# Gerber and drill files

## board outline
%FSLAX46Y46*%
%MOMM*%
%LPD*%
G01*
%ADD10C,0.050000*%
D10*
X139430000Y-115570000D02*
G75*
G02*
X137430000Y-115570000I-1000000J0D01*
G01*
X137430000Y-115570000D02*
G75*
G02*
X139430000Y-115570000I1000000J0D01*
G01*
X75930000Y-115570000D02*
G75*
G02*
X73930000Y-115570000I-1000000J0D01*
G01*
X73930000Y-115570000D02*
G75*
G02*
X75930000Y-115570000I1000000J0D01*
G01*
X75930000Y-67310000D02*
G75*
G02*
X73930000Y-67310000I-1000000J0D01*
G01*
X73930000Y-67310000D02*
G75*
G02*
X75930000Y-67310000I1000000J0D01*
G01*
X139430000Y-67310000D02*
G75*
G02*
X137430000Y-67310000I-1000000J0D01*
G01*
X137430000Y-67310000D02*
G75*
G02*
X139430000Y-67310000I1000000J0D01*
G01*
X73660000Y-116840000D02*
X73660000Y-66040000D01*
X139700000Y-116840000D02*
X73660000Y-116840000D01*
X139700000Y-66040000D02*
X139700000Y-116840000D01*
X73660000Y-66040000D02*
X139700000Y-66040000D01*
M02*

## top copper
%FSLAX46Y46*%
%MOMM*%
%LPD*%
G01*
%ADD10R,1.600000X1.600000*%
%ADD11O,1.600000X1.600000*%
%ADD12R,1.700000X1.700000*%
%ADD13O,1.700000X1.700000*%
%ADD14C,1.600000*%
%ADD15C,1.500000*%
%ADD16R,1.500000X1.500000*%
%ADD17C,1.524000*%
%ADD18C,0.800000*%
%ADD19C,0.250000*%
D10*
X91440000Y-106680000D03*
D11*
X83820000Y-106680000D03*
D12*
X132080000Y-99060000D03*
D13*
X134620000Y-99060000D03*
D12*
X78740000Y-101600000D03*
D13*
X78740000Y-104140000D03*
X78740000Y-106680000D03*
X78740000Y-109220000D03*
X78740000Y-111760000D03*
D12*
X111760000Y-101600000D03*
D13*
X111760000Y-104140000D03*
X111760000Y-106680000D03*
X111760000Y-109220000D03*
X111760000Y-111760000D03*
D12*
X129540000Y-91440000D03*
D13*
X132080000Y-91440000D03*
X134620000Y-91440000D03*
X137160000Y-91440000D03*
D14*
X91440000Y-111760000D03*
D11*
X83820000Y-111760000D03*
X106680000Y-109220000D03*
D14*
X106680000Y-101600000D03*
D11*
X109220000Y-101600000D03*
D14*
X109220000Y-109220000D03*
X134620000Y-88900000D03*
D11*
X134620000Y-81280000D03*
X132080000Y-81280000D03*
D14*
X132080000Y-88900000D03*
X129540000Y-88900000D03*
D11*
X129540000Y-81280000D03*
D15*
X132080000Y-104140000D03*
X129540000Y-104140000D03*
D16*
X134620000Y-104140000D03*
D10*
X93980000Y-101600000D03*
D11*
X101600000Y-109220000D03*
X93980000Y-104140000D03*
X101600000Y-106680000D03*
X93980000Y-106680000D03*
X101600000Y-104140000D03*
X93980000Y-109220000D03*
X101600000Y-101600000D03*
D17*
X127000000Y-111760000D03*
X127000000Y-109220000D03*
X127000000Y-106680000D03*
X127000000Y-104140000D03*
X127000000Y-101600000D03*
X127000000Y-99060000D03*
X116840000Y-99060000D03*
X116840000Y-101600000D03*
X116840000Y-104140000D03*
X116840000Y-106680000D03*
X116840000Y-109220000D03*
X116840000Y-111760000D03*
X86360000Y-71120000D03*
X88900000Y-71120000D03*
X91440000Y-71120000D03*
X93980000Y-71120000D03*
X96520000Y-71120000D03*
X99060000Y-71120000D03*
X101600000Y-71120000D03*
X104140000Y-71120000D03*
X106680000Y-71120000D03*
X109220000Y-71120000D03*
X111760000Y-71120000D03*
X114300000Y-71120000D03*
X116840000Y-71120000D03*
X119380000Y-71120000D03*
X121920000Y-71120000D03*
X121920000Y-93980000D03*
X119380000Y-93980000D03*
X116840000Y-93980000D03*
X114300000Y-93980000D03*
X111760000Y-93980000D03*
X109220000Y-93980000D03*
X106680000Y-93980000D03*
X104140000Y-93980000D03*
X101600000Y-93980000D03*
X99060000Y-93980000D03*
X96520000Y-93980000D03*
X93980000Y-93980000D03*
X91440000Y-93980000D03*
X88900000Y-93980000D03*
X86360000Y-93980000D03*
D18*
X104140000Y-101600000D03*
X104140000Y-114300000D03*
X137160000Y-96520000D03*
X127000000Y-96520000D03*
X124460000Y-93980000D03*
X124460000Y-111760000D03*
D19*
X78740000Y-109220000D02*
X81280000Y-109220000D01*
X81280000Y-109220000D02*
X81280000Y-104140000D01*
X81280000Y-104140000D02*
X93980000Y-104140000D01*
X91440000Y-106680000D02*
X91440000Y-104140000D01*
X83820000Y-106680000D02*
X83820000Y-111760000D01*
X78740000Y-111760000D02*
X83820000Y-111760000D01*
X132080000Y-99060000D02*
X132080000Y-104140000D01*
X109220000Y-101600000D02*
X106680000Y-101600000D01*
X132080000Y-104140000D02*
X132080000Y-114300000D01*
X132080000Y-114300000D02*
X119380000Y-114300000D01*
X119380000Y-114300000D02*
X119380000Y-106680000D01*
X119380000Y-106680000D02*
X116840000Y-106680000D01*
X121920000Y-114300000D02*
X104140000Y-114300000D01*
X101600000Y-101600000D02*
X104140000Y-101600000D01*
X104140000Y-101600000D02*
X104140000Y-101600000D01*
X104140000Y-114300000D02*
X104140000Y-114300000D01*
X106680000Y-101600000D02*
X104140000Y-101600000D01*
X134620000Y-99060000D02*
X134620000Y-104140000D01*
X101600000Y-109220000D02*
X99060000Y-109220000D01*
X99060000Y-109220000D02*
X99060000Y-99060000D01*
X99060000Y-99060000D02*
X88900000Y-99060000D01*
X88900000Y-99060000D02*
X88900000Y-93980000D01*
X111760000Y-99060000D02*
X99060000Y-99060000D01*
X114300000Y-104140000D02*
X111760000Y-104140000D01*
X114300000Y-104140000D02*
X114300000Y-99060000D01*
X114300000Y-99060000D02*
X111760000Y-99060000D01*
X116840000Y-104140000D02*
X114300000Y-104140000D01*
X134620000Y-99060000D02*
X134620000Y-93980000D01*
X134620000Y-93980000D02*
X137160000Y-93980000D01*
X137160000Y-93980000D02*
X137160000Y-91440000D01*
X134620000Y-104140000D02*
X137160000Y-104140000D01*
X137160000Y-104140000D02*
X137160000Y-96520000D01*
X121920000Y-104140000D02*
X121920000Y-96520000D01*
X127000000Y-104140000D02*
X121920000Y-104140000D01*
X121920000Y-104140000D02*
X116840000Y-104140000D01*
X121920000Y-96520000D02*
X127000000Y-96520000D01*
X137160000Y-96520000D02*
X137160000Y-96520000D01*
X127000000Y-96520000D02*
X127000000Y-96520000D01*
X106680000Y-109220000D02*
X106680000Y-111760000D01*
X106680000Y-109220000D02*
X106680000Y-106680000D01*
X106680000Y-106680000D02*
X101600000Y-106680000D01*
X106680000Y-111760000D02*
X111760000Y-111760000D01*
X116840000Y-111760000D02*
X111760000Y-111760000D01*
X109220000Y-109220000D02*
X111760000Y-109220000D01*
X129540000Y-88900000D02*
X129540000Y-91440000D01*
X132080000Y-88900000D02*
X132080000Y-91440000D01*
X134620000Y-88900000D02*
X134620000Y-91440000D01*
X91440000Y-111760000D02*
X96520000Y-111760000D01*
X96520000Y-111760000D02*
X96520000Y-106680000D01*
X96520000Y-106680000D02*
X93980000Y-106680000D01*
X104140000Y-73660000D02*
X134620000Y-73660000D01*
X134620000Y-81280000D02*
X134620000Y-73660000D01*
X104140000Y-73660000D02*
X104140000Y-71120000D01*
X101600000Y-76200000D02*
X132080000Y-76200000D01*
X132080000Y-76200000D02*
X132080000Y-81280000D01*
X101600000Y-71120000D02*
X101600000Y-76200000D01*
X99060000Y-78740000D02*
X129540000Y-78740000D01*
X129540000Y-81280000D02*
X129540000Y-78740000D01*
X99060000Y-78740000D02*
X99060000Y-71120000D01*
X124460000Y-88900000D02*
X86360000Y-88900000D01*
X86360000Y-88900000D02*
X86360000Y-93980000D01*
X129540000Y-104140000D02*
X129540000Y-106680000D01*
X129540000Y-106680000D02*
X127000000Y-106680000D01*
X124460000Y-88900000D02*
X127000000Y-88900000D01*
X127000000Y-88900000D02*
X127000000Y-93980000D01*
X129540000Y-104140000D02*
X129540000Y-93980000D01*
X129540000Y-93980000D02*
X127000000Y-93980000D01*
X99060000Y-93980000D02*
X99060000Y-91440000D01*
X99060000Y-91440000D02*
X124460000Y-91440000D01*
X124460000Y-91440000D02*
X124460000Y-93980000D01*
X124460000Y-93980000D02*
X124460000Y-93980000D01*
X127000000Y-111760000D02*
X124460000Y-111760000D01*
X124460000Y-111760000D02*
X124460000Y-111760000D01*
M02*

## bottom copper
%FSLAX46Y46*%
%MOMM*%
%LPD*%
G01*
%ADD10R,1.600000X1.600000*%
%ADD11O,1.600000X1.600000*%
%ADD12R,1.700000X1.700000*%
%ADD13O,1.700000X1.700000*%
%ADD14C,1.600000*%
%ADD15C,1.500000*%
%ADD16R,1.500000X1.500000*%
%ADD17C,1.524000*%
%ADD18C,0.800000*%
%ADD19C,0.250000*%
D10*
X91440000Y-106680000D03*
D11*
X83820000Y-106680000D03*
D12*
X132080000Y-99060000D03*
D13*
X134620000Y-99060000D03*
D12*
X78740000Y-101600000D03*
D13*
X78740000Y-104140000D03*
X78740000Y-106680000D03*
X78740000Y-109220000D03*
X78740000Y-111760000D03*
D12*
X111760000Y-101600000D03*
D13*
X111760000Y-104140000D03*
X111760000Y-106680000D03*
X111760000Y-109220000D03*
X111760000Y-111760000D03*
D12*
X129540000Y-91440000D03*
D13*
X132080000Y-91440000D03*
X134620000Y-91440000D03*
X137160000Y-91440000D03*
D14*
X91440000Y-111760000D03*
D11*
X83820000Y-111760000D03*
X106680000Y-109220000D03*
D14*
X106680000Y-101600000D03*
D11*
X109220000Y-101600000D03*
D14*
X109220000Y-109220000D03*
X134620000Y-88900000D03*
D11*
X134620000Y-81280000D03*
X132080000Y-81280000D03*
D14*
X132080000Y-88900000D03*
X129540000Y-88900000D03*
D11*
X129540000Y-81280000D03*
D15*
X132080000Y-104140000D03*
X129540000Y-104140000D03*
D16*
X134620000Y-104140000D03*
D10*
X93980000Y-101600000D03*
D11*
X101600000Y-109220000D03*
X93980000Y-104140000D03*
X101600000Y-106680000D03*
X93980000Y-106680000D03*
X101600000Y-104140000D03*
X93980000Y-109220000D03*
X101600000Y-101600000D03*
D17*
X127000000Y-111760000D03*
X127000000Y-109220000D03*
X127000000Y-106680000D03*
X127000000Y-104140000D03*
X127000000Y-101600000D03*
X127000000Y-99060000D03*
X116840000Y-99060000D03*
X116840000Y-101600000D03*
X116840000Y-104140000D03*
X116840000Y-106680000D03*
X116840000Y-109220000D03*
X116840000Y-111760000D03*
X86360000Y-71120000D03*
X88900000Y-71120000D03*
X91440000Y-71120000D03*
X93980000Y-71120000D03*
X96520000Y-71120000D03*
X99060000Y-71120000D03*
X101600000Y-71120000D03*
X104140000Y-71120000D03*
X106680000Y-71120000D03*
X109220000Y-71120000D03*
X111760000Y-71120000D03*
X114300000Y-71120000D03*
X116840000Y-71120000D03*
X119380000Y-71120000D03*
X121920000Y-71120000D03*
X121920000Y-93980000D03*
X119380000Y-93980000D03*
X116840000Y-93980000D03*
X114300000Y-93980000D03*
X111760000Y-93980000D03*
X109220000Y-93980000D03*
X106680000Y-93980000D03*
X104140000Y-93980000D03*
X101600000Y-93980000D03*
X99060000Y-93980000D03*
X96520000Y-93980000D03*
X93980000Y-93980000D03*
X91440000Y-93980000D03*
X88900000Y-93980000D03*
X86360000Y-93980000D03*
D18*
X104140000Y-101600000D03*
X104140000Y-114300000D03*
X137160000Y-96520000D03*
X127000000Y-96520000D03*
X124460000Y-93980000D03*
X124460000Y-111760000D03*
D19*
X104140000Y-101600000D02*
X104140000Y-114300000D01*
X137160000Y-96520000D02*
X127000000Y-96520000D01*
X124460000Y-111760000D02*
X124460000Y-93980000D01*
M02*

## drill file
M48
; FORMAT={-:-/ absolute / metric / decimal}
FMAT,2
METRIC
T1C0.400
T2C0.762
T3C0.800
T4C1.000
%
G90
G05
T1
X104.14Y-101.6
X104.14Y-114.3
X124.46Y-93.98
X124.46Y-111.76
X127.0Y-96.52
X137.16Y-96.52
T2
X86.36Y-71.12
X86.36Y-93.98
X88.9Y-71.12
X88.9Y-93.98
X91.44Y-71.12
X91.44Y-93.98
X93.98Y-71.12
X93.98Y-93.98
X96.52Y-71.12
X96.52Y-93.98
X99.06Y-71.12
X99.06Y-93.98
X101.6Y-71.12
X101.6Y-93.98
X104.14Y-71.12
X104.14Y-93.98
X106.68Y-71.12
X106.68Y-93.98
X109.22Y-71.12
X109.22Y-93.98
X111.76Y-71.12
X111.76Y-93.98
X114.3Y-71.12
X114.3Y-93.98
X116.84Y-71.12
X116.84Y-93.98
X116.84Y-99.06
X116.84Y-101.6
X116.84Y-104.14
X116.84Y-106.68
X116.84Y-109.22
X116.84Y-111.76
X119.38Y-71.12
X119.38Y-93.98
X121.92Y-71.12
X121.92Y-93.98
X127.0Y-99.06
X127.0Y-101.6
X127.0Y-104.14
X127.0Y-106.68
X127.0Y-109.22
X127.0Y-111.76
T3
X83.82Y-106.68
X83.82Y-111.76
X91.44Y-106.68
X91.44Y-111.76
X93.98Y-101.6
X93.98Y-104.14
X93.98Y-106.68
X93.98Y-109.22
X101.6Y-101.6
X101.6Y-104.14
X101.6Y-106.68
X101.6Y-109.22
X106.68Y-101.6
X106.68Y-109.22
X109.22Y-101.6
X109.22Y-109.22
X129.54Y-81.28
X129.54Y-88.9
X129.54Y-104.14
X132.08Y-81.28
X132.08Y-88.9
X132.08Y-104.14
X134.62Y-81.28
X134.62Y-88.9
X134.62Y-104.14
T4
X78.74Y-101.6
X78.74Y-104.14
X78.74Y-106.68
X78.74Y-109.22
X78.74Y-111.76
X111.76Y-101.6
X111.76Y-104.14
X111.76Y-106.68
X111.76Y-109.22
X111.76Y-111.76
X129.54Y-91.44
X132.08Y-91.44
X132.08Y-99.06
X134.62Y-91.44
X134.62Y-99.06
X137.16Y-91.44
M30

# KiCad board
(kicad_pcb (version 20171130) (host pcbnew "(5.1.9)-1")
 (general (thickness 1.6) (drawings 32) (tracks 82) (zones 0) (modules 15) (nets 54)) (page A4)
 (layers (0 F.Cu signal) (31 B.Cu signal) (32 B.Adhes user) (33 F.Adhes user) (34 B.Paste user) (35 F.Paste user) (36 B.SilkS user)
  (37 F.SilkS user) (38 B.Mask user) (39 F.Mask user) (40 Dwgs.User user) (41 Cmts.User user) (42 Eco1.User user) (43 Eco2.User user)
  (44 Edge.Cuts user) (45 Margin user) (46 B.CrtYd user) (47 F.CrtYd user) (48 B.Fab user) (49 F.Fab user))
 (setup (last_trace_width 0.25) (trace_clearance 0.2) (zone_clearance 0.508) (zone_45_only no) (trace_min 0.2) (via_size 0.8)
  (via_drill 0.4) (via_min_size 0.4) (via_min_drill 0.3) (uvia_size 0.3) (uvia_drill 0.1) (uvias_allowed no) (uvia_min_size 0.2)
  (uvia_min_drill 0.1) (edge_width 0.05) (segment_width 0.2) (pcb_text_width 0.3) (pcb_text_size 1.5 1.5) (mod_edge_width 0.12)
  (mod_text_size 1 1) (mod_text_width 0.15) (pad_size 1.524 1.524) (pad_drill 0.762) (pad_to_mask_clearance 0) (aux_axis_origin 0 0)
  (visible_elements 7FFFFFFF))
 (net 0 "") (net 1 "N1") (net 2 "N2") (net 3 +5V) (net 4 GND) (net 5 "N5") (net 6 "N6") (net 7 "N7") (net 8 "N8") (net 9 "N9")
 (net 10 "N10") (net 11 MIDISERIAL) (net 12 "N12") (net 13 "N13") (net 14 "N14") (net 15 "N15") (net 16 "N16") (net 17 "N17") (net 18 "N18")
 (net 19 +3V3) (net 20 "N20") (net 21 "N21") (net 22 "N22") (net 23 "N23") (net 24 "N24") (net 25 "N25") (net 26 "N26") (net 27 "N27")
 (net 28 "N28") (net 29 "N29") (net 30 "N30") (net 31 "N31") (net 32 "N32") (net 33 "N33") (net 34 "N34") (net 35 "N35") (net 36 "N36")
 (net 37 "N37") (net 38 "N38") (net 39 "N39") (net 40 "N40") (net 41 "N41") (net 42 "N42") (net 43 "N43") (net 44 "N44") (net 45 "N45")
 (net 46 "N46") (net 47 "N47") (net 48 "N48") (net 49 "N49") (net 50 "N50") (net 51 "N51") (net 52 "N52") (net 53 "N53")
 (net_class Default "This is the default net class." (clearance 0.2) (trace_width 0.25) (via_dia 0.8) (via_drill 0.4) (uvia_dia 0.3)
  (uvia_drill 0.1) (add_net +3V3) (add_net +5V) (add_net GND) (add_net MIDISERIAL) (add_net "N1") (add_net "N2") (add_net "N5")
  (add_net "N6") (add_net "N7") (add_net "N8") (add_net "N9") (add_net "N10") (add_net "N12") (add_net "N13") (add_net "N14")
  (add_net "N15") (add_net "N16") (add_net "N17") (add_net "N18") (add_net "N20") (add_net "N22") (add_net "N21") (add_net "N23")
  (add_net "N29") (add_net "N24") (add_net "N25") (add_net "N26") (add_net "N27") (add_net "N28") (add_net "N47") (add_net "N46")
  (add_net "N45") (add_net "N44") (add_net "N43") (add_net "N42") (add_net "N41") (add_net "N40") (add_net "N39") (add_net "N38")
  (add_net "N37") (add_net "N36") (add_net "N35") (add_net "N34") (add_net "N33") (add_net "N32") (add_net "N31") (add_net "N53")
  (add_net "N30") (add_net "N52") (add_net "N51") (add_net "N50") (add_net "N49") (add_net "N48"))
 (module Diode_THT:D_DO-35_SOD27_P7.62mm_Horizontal (layer F.Cu) (at 91.44 106.68 180)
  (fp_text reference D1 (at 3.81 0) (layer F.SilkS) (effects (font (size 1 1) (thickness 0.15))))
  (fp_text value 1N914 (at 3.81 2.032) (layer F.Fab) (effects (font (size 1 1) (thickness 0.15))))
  (pad 1 thru_hole rect (at 0 0 180) (size 1.6 1.6) (drill 0.8) (layers *.Cu *.Mask) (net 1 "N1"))
  (pad 2 thru_hole oval (at 7.62 0 180) (size 1.6 1.6) (drill 0.8) (layers *.Cu *.Mask) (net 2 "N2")))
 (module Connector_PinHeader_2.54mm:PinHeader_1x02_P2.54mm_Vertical (layer F.Cu) (at 132.08 99.06 90)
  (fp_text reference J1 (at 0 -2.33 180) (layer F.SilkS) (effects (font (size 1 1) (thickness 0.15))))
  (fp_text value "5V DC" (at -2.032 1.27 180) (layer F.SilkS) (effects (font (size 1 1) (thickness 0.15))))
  (pad 1 thru_hole rect (at 0 0 90) (size 1.7 1.7) (drill 1) (layers *.Cu *.Mask) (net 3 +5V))
  (pad 2 thru_hole oval (at 0 2.54 90) (size 1.7 1.7) (drill 1) (layers *.Cu *.Mask) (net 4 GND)))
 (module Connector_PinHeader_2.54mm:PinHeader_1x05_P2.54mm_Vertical (layer F.Cu) (at 78.74 101.6)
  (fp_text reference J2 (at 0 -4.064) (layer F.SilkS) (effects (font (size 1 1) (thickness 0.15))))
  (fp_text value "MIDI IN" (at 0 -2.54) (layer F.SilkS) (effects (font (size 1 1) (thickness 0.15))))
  (pad 1 thru_hole rect (at 0 0) (size 1.7 1.7) (drill 1) (layers *.Cu *.Mask) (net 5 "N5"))
  (pad 2 thru_hole oval (at 0 2.54) (size 1.7 1.7) (drill 1) (layers *.Cu *.Mask) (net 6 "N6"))
  (pad 3 thru_hole oval (at 0 5.08) (size 1.7 1.7) (drill 1) (layers *.Cu *.Mask) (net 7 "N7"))
  (pad 4 thru_hole oval (at 0 7.62) (size 1.7 1.7) (drill 1) (layers *.Cu *.Mask) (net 1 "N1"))
  (pad 5 thru_hole oval (at 0 10.16) (size 1.7 1.7) (drill 1) (layers *.Cu *.Mask) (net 2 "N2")))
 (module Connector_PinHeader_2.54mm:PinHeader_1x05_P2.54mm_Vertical (layer F.Cu) (at 111.76 101.6)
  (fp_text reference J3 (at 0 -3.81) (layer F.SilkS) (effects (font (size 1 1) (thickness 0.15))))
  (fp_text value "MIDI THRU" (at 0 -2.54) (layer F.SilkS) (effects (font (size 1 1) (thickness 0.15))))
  (pad 1 thru_hole rect (at 0 0) (size 1.7 1.7) (drill 1) (layers *.Cu *.Mask) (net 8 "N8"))
  (pad 2 thru_hole oval (at 0 2.54) (size 1.7 1.7) (drill 1) (layers *.Cu *.Mask) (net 4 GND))
  (pad 3 thru_hole oval (at 0 5.08) (size 1.7 1.7) (drill 1) (layers *.Cu *.Mask) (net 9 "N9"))
  (pad 4 thru_hole oval (at 0 7.62) (size 1.7 1.7) (drill 1) (layers *.Cu *.Mask) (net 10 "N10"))
  (pad 5 thru_hole oval (at 0 10.16) (size 1.7 1.7) (drill 1) (layers *.Cu *.Mask) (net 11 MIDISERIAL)))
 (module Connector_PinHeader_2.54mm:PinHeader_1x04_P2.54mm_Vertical (layer F.Cu) (at 129.54 91.44 90)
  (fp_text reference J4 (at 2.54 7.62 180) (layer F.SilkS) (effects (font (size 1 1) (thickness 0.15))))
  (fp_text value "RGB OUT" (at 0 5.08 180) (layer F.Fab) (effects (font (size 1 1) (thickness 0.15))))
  (pad 1 thru_hole rect (at 0 0 90) (size 1.7 1.7) (drill 1) (layers *.Cu *.Mask) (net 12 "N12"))
  (pad 2 thru_hole oval (at 0 2.54 90) (size 1.7 1.7) (drill 1) (layers *.Cu *.Mask) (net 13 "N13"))
  (pad 3 thru_hole oval (at 0 5.08 90) (size 1.7 1.7) (drill 1) (layers *.Cu *.Mask) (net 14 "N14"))
  (pad 4 thru_hole oval (at 0 7.62 90) (size 1.7 1.7) (drill 1) (layers *.Cu *.Mask) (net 4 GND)))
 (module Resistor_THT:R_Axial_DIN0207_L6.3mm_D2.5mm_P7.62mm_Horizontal (layer F.Cu) (at 91.44 111.76 180)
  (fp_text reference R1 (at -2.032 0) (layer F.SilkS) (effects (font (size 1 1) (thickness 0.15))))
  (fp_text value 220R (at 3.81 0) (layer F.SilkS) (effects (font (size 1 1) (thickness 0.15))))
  (pad 1 thru_hole circle (at 0 0 180) (size 1.6 1.6) (drill 0.8) (layers *.Cu *.Mask) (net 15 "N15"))
  (pad 2 thru_hole oval (at 7.62 0 180) (size 1.6 1.6) (drill 0.8) (layers *.Cu *.Mask) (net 2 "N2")))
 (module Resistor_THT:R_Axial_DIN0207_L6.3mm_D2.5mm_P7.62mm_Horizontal (layer F.Cu) (at 106.68 101.6 270)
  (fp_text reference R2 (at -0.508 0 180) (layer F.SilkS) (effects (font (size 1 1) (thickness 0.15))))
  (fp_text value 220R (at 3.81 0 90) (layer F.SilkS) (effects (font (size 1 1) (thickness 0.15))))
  (pad 2 thru_hole oval (at 7.62 0 270) (size 1.6 1.6) (drill 0.8) (layers *.Cu *.Mask) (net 11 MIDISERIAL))
  (pad 1 thru_hole circle (at 0 0 270) (size 1.6 1.6) (drill 0.8) (layers *.Cu *.Mask) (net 3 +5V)))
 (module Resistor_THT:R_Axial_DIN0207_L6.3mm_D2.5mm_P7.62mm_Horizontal (layer F.Cu) (at 109.22 109.22 90)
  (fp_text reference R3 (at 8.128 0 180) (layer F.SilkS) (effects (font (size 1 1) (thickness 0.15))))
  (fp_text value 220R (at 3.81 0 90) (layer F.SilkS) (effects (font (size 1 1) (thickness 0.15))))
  (pad 2 thru_hole oval (at 7.62 0 90) (size 1.6 1.6) (drill 0.8) (layers *.Cu *.Mask) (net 3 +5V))
  (pad 1 thru_hole circle (at 0 0 90) (size 1.6 1.6) (drill 0.8) (layers *.Cu *.Mask) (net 10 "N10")))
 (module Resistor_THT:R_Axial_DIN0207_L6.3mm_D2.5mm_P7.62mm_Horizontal (layer F.Cu) (at 134.62 88.9 90)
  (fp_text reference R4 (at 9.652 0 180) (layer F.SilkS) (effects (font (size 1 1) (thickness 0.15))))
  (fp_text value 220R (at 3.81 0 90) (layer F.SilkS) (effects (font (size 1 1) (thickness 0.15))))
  (pad 1 thru_hole circle (at 0 0 90) (size 1.6 1.6) (drill 0.8) (layers *.Cu *.Mask) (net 14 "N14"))
  (pad 2 thru_hole oval (at 7.62 0 90) (size 1.6 1.6) (drill 0.8) (layers *.Cu *.Mask) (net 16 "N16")))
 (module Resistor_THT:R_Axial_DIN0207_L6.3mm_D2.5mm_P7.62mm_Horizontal (layer F.Cu) (at 132.08 88.9 90)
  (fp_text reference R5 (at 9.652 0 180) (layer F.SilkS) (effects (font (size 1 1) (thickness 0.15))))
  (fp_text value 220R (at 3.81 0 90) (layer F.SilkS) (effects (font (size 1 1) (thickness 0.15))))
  (pad 2 thru_hole oval (at 7.62 0 90) (size 1.6 1.6) (drill 0.8) (layers *.Cu *.Mask) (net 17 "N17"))
  (pad 1 thru_hole circle (at 0 0 90) (size 1.6 1.6) (drill 0.8) (layers *.Cu *.Mask) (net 13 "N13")))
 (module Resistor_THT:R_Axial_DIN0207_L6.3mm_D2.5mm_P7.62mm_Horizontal (layer F.Cu) (at 129.54 88.9 90)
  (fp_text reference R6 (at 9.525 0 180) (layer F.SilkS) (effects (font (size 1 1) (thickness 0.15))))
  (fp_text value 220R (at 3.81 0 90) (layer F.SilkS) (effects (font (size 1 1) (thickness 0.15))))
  (pad 1 thru_hole circle (at 0 0 90) (size 1.6 1.6) (drill 0.8) (layers *.Cu *.Mask) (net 12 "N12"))
  (pad 2 thru_hole oval (at 7.62 0 90) (size 1.6 1.6) (drill 0.8) (layers *.Cu *.Mask) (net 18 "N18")))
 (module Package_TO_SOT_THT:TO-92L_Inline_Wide (layer F.Cu) (at 134.62 104.14 180)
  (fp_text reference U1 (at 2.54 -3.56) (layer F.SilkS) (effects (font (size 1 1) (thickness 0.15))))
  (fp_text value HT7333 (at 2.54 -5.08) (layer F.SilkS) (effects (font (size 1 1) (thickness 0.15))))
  (pad 2 thru_hole circle (at 2.54 0 180) (size 1.5 1.5) (drill 0.8) (layers *.Cu *.Mask) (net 3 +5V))
  (pad 3 thru_hole circle (at 5.08 0 180) (size 1.5 1.5) (drill 0.8) (layers *.Cu *.Mask) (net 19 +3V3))
  (pad 1 thru_hole rect (at 0 0 180) (size 1.5 1.5) (drill 0.8) (layers *.Cu *.Mask) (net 4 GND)))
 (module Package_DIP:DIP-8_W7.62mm (layer F.Cu) (at 93.98 101.6)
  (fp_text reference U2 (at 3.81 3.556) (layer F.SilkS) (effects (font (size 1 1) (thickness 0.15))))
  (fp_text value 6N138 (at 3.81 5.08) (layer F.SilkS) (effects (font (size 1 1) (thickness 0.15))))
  (pad 1 thru_hole rect (at 0 0) (size 1.6 1.6) (drill 0.8) (layers *.Cu *.Mask) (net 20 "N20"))
  (pad 5 thru_hole oval (at 7.62 7.62) (size 1.6 1.6) (drill 0.8) (layers *.Cu *.Mask) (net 4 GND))
  (pad 2 thru_hole oval (at 0 2.54) (size 1.6 1.6) (drill 0.8) (layers *.Cu *.Mask) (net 1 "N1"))
  (pad 6 thru_hole oval (at 7.62 5.08) (size 1.6 1.6) (drill 0.8) (layers *.Cu *.Mask) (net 11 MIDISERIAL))
  (pad 3 thru_hole oval (at 0 5.08) (size 1.6 1.6) (drill 0.8) (layers *.Cu *.Mask) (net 15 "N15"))
  (pad 7 thru_hole oval (at 7.62 2.54) (size 1.6 1.6) (drill 0.8) (layers *.Cu *.Mask) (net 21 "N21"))
  (pad 4 thru_hole oval (at 0 7.62) (size 1.6 1.6) (drill 0.8) (layers *.Cu *.Mask) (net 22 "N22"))
  (pad 8 thru_hole oval (at 7.62 0) (size 1.6 1.6) (drill 0.8) (layers *.Cu *.Mask) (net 3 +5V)))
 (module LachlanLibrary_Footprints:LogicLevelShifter (layer F.Cu) (at 121.92 105.41 180)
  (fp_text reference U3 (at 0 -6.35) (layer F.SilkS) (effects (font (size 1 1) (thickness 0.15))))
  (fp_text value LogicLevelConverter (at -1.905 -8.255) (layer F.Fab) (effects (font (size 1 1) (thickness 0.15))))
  (pad 1 thru_hole circle (at -5.08 -6.35 180) (size 1.524 1.524) (drill 0.762) (layers *.Cu *.Mask) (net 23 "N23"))
  (pad 2 thru_hole circle (at -5.08 -3.81 180) (size 1.524 1.524) (drill 0.762) (layers *.Cu *.Mask) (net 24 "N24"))
  (pad 3 thru_hole circle (at -5.08 -1.27 180) (size 1.524 1.524) (drill 0.762) (layers *.Cu *.Mask) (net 19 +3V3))
  (pad 4 thru_hole circle (at -5.08 1.27 180) (size 1.524 1.524) (drill 0.762) (layers *.Cu *.Mask) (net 4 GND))
  (pad 5 thru_hole circle (at -5.08 3.81 180) (size 1.524 1.524) (drill 0.762) (layers *.Cu *.Mask) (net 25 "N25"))
  (pad 6 thru_hole circle (at -5.08 6.35 180) (size 1.524 1.524) (drill 0.762) (layers *.Cu *.Mask) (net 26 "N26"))
  (pad 7 thru_hole circle (at 5.08 6.35 180) (size 1.524 1.524) (drill 0.762) (layers *.Cu *.Mask) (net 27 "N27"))
  (pad 8 thru_hole circle (at 5.08 3.81 180) (size 1.524 1.524) (drill 0.762) (layers *.Cu *.Mask) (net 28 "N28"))
  (pad 9 thru_hole circle (at 5.08 1.27 180) (size 1.524 1.524) (drill 0.762) (layers *.Cu *.Mask) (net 4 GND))
  (pad 10 thru_hole circle (at 5.08 -1.27 180) (size 1.524 1.524) (drill 0.762) (layers *.Cu *.Mask) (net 3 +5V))
  (pad 11 thru_hole circle (at 5.08 -3.81 180) (size 1.524 1.524) (drill 0.762) (layers *.Cu *.Mask) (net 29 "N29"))
  (pad 12 thru_hole circle (at 5.08 -6.35 180) (size 1.524 1.524) (drill 0.762) (layers *.Cu *.Mask) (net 11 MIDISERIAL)))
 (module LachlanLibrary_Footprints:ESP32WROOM (layer F.Cu) (at 105.41 82.55 90)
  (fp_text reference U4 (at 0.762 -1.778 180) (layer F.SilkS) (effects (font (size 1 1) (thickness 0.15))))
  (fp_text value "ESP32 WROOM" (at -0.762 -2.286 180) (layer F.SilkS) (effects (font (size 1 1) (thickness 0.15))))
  (pad 30 thru_hole circle (at 11.43 -19.05 90) (size 1.524 1.524) (drill 0.762) (layers *.Cu *.Mask) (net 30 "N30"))
  (pad 29 thru_hole circle (at 11.43 -16.51 90) (size 1.524 1.524) (drill 0.762) (layers *.Cu *.Mask) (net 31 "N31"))
  (pad 28 thru_hole circle (at 11.43 -13.97 90) (size 1.524 1.524) (drill 0.762) (layers *.Cu *.Mask) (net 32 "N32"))
  (pad 27 thru_hole circle (at 11.43 -11.43 90) (size 1.524 1.524) (drill 0.762) (layers *.Cu *.Mask) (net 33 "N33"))
  (pad 26 thru_hole circle (at 11.43 -8.89 90) (size 1.524 1.524) (drill 0.762) (layers *.Cu *.Mask) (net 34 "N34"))
  (pad 25 thru_hole circle (at 11.43 -6.35 90) (size 1.524 1.524) (drill 0.762) (layers *.Cu *.Mask) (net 18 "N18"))
  (pad 24 thru_hole circle (at 11.43 -3.81 90) (size 1.524 1.524) (drill 0.762) (layers *.Cu *.Mask) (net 17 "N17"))
  (pad 23 thru_hole circle (at 11.43 -1.27 90) (size 1.524 1.524) (drill 0.762) (layers *.Cu *.Mask) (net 16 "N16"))
  (pad 22 thru_hole circle (at 11.43 1.27 90) (size 1.524 1.524) (drill 0.762) (layers *.Cu *.Mask) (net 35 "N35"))
  (pad 21 thru_hole circle (at 11.43 3.81 90) (size 1.524 1.524) (drill 0.762) (layers *.Cu *.Mask) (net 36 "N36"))
  (pad 20 thru_hole circle (at 11.43 6.35 90) (size 1.524 1.524) (drill 0.762) (layers *.Cu *.Mask) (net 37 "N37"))
  (pad 19 thru_hole circle (at 11.43 8.89 90) (size 1.524 1.524) (drill 0.762) (layers *.Cu *.Mask) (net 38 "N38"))
  (pad 18 thru_hole circle (at 11.43 11.43 90) (size 1.524 1.524) (drill 0.762) (layers *.Cu *.Mask) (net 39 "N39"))
  (pad 17 thru_hole circle (at 11.43 13.97 90) (size 1.524 1.524) (drill 0.762) (layers *.Cu *.Mask) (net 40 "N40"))
  (pad 16 thru_hole circle (at 11.43 16.51 90) (size 1.524 1.524) (drill 0.762) (layers *.Cu *.Mask) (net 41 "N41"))
  (pad 15 thru_hole circle (at -11.43 16.51 90) (size 1.524 1.524) (drill 0.762) (layers *.Cu *.Mask) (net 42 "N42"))
  (pad 14 thru_hole circle (at -11.43 13.97 90) (size 1.524 1.524) (drill 0.762) (layers *.Cu *.Mask) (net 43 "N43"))
  (pad 13 thru_hole circle (at -11.43 11.43 90) (size 1.524 1.524) (drill 0.762) (layers *.Cu *.Mask) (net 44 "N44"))
  (pad 12 thru_hole circle (at -11.43 8.89 90) (size 1.524 1.524) (drill 0.762) (layers *.Cu *.Mask) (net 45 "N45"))
  (pad 11 thru_hole circle (at -11.43 6.35 90) (size 1.524 1.524) (drill 0.762) (layers *.Cu *.Mask) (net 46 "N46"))
  (pad 10 thru_hole circle (at -11.43 3.81 90) (size 1.524 1.524) (drill 0.762) (layers *.Cu *.Mask) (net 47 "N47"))
  (pad 9 thru_hole circle (at -11.43 1.27 90) (size 1.524 1.524) (drill 0.762) (layers *.Cu *.Mask) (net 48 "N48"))
  (pad 8 thru_hole circle (at -11.43 -1.27 90) (size 1.524 1.524) (drill 0.762) (layers *.Cu *.Mask) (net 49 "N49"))
  (pad 7 thru_hole circle (at -11.43 -3.81 90) (size 1.524 1.524) (drill 0.762) (layers *.Cu *.Mask) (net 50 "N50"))
  (pad 6 thru_hole circle (at -11.43 -6.35 90) (size 1.524 1.524) (drill 0.762) (layers *.Cu *.Mask) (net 23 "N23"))
  (pad 5 thru_hole circle (at -11.43 -8.89 90) (size 1.524 1.524) (drill 0.762) (layers *.Cu *.Mask) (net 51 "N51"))
  (pad 4 thru_hole circle (at -11.43 -11.43 90) (size 1.524 1.524) (drill 0.762) (layers *.Cu *.Mask) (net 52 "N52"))
  (pad 3 thru_hole circle (at -11.43 -13.97 90) (size 1.524 1.524) (drill 0.762) (layers *.Cu *.Mask) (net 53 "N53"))
  (pad 2 thru_hole circle (at -11.43 -16.51 90) (size 1.524 1.524) (drill 0.762) (layers *.Cu *.Mask) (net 4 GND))
  (pad 1 thru_hole circle (at -11.43 -19.05 90) (size 1.524 1.524) (drill 0.762) (layers *.Cu *.Mask) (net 19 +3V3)))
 (gr_circle (center 138.43 115.57) (end 139.43 115.57) (layer Edge.Cuts) (width 0.05))
 (gr_circle (center 74.93 115.57) (end 75.93 115.57) (layer Edge.Cuts) (width 0.05))
 (gr_circle (center 74.93 67.31) (end 75.93 67.31) (layer Edge.Cuts) (width 0.05))
 (gr_circle (center 138.43 67.31) (end 139.43 67.31) (layer Edge.Cuts) (width 0.05))
 (gr_line (start 73.66 116.84) (end 73.66 66.04) (layer Edge.Cuts) (width 0.05))
 (gr_line (start 139.7 116.84) (end 73.66 116.84) (layer Edge.Cuts) (width 0.05))
 (gr_line (start 139.7 66.04) (end 139.7 116.84) (layer Edge.Cuts) (width 0.05))
 (gr_line (start 73.66 66.04) (end 139.7 66.04) (layer Edge.Cuts) (width 0.05))
 (segment (start 78.74 109.22) (end 81.28 109.22) (width 0.25) (layer F.Cu) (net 1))
 (segment (start 81.28 109.22) (end 81.28 104.14) (width 0.25) (layer F.Cu) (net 1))
 (segment (start 81.28 104.14) (end 93.98 104.14) (width 0.25) (layer F.Cu) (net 1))
 (segment (start 91.44 106.68) (end 91.44 104.14) (width 0.25) (layer F.Cu) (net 1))
 (segment (start 83.82 106.68) (end 83.82 111.76) (width 0.25) (layer F.Cu) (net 2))
 (segment (start 78.74 111.76) (end 83.82 111.76) (width 0.25) (layer F.Cu) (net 2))
 (segment (start 132.08 99.06) (end 132.08 104.14) (width 0.25) (layer F.Cu) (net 3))
 (segment (start 109.22 101.6) (end 106.68 101.6) (width 0.25) (layer F.Cu) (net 3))
 (segment (start 132.08 104.14) (end 132.08 114.3) (width 0.25) (layer F.Cu) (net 3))
 (segment (start 132.08 114.3) (end 119.38 114.3) (width 0.25) (layer F.Cu) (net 3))
 (segment (start 119.38 114.3) (end 119.38 106.68) (width 0.25) (layer F.Cu) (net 3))
 (segment (start 119.38 106.68) (end 116.84 106.68) (width 0.25) (layer F.Cu) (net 3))
 (segment (start 121.92 114.3) (end 104.14 114.3) (width 0.25) (layer F.Cu) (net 3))
 (segment (start 101.6 101.6) (end 104.14 101.6) (width 0.25) (layer F.Cu) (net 3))
 (segment (start 104.14 101.6) (end 104.14 101.6) (width 0.25) (layer F.Cu) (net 3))
 (via (at 104.14 101.6) (size 0.8) (drill 0.4) (layers F.Cu B.Cu) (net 3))
 (segment (start 104.14 114.3) (end 104.14 114.3) (width 0.25) (layer F.Cu) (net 3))
 (via (at 104.14 114.3) (size 0.8) (drill 0.4) (layers F.Cu B.Cu) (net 3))
 (segment (start 106.68 101.6) (end 104.14 101.6) (width 0.25) (layer F.Cu) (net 3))
 (segment (start 104.14 101.6) (end 104.14 114.3) (width 0.25) (layer B.Cu) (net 3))
 (segment (start 134.62 99.06) (end 134.62 104.14) (width 0.25) (layer F.Cu) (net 4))
 (segment (start 101.6 109.22) (end 99.06 109.22) (width 0.25) (layer F.Cu) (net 4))
 (segment (start 99.06 109.22) (end 99.06 99.06) (width 0.25) (layer F.Cu) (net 4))
 (segment (start 99.06 99.06) (end 88.9 99.06) (width 0.25) (layer F.Cu) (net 4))
 (segment (start 88.9 99.06) (end 88.9 93.98) (width 0.25) (layer F.Cu) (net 4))
 (segment (start 111.76 99.06) (end 99.06 99.06) (width 0.25) (layer F.Cu) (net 4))
 (segment (start 114.3 104.14) (end 111.76 104.14) (width 0.25) (layer F.Cu) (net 4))
 (segment (start 114.3 104.14) (end 114.3 99.06) (width 0.25) (layer F.Cu) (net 4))
 (segment (start 114.3 99.06) (end 111.76 99.06) (width 0.25) (layer F.Cu) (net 4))
 (segment (start 116.84 104.14) (end 114.3 104.14) (width 0.25) (layer F.Cu) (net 4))
 (segment (start 134.62 99.06) (end 134.62 93.98) (width 0.25) (layer F.Cu) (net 4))
 (segment (start 134.62 93.98) (end 137.16 93.98) (width 0.25) (layer F.Cu) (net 4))
 (segment (start 137.16 93.98) (end 137.16 91.44) (width 0.25) (layer F.Cu) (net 4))
 (segment (start 134.62 104.14) (end 137.16 104.14) (width 0.25) (layer F.Cu) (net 4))
 (segment (start 137.16 104.14) (end 137.16 96.52) (width 0.25) (layer F.Cu) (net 4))
 (segment (start 121.92 104.14) (end 121.92 96.52) (width 0.25) (layer F.Cu) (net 4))
 (segment (start 127 104.14) (end 121.92 104.14) (width 0.25) (layer F.Cu) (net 4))
 (segment (start 121.92 104.14) (end 116.84 104.14) (width 0.25) (layer F.Cu) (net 4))
 (segment (start 121.92 96.52) (end 127 96.52) (width 0.25) (layer F.Cu) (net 4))
 (segment (start 137.16 96.52) (end 137.16 96.52) (width 0.25) (layer F.Cu) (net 4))
 (via (at 137.16 96.52) (size 0.8) (drill 0.4) (layers F.Cu B.Cu) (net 4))
 (segment (start 127 96.52) (end 127 96.52) (width 0.25) (layer F.Cu) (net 4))
 (via (at 127 96.52) (size 0.8) (drill 0.4) (layers F.Cu B.Cu) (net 4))
 (segment (start 137.16 96.52) (end 127 96.52) (width 0.25) (layer B.Cu) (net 4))
 (segment (start 106.68 109.22) (end 106.68 111.76) (width 0.25) (layer F.Cu) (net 11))
 (segment (start 106.68 109.22) (end 106.68 106.68) (width 0.25) (layer F.Cu) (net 11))
 (segment (start 106.68 106.68) (end 101.6 106.68) (width 0.25) (layer F.Cu) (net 11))
 (segment (start 106.68 111.76) (end 111.76 111.76) (width 0.25) (layer F.Cu) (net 11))
 (segment (start 116.84 111.76) (end 111.76 111.76) (width 0.25) (layer F.Cu) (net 11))
 (segment (start 109.22 109.22) (end 111.76 109.22) (width 0.25) (layer F.Cu) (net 10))
 (segment (start 129.54 88.9) (end 129.54 91.44) (width 0.25) (layer F.Cu) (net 12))
 (segment (start 132.08 88.9) (end 132.08 91.44) (width 0.25) (layer F.Cu) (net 13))
 (segment (start 134.62 88.9) (end 134.62 91.44) (width 0.25) (layer F.Cu) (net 14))
 (segment (start 91.44 111.76) (end 96.52 111.76) (width 0.25) (layer F.Cu) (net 15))
 (segment (start 96.52 111.76) (end 96.52 106.68) (width 0.25) (layer F.Cu) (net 15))
 (segment (start 96.52 106.68) (end 93.98 106.68) (width 0.25) (layer F.Cu) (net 15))
 (segment (start 104.14 73.66) (end 134.62 73.66) (width 0.25) (layer F.Cu) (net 16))
 (segment (start 134.62 81.28) (end 134.62 73.66) (width 0.25) (layer F.Cu) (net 16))
 (segment (start 104.14 73.66) (end 104.14 71.12) (width 0.25) (layer F.Cu) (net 16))
 (segment (start 101.6 76.2) (end 132.08 76.2) (width 0.25) (layer F.Cu) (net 17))
 (segment (start 132.08 76.2) (end 132.08 81.28) (width 0.25) (layer F.Cu) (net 17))
 (segment (start 101.6 71.12) (end 101.6 76.2) (width 0.25) (layer F.Cu) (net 17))
 (segment (start 99.06 78.74) (end 129.54 78.74) (width 0.25) (layer F.Cu) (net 18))
 (segment (start 129.54 81.28) (end 129.54 78.74) (width 0.25) (layer F.Cu) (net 18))
 (segment (start 99.06 78.74) (end 99.06 71.12) (width 0.25) (layer F.Cu) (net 18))
 (segment (start 124.46 88.9) (end 86.36 88.9) (width 0.25) (layer F.Cu) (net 19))
 (segment (start 86.36 88.9) (end 86.36 93.98) (width 0.25) (layer F.Cu) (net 19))
 (segment (start 129.54 104.14) (end 129.54 106.68) (width 0.25) (layer F.Cu) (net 19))
 (segment (start 129.54 106.68) (end 127 106.68) (width 0.25) (layer F.Cu) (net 19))
 (segment (start 124.46 88.9) (end 127 88.9) (width 0.25) (layer F.Cu) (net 19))
 (segment (start 127 88.9) (end 127 93.98) (width 0.25) (layer F.Cu) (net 19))
 (segment (start 129.54 104.14) (end 129.54 93.98) (width 0.25) (layer F.Cu) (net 19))
 (segment (start 129.54 93.98) (end 127 93.98) (width 0.25) (layer F.Cu) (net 19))
 (segment (start 99.06 93.98) (end 99.06 91.44) (width 0.25) (layer F.Cu) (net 23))
 (segment (start 99.06 91.44) (end 124.46 91.44) (width 0.25) (layer F.Cu) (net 23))
 (segment (start 124.46 91.44) (end 124.46 93.98) (width 0.25) (layer F.Cu) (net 23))
 (segment (start 124.46 93.98) (end 124.46 93.98) (width 0.25) (layer F.Cu) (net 23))
 (via (at 124.46 93.98) (size 0.8) (drill 0.4) (layers F.Cu B.Cu) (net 23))
 (segment (start 127 111.76) (end 124.46 111.76) (width 0.25) (layer F.Cu) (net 23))
 (segment (start 124.46 111.76) (end 124.46 111.76) (width 0.25) (layer F.Cu) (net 23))
 (via (at 124.46 111.76) (size 0.8) (drill 0.4) (layers F.Cu B.Cu) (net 23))
 (segment (start 124.46 111.76) (end 124.46 93.98) (width 0.25) (layer B.Cu) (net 23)))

